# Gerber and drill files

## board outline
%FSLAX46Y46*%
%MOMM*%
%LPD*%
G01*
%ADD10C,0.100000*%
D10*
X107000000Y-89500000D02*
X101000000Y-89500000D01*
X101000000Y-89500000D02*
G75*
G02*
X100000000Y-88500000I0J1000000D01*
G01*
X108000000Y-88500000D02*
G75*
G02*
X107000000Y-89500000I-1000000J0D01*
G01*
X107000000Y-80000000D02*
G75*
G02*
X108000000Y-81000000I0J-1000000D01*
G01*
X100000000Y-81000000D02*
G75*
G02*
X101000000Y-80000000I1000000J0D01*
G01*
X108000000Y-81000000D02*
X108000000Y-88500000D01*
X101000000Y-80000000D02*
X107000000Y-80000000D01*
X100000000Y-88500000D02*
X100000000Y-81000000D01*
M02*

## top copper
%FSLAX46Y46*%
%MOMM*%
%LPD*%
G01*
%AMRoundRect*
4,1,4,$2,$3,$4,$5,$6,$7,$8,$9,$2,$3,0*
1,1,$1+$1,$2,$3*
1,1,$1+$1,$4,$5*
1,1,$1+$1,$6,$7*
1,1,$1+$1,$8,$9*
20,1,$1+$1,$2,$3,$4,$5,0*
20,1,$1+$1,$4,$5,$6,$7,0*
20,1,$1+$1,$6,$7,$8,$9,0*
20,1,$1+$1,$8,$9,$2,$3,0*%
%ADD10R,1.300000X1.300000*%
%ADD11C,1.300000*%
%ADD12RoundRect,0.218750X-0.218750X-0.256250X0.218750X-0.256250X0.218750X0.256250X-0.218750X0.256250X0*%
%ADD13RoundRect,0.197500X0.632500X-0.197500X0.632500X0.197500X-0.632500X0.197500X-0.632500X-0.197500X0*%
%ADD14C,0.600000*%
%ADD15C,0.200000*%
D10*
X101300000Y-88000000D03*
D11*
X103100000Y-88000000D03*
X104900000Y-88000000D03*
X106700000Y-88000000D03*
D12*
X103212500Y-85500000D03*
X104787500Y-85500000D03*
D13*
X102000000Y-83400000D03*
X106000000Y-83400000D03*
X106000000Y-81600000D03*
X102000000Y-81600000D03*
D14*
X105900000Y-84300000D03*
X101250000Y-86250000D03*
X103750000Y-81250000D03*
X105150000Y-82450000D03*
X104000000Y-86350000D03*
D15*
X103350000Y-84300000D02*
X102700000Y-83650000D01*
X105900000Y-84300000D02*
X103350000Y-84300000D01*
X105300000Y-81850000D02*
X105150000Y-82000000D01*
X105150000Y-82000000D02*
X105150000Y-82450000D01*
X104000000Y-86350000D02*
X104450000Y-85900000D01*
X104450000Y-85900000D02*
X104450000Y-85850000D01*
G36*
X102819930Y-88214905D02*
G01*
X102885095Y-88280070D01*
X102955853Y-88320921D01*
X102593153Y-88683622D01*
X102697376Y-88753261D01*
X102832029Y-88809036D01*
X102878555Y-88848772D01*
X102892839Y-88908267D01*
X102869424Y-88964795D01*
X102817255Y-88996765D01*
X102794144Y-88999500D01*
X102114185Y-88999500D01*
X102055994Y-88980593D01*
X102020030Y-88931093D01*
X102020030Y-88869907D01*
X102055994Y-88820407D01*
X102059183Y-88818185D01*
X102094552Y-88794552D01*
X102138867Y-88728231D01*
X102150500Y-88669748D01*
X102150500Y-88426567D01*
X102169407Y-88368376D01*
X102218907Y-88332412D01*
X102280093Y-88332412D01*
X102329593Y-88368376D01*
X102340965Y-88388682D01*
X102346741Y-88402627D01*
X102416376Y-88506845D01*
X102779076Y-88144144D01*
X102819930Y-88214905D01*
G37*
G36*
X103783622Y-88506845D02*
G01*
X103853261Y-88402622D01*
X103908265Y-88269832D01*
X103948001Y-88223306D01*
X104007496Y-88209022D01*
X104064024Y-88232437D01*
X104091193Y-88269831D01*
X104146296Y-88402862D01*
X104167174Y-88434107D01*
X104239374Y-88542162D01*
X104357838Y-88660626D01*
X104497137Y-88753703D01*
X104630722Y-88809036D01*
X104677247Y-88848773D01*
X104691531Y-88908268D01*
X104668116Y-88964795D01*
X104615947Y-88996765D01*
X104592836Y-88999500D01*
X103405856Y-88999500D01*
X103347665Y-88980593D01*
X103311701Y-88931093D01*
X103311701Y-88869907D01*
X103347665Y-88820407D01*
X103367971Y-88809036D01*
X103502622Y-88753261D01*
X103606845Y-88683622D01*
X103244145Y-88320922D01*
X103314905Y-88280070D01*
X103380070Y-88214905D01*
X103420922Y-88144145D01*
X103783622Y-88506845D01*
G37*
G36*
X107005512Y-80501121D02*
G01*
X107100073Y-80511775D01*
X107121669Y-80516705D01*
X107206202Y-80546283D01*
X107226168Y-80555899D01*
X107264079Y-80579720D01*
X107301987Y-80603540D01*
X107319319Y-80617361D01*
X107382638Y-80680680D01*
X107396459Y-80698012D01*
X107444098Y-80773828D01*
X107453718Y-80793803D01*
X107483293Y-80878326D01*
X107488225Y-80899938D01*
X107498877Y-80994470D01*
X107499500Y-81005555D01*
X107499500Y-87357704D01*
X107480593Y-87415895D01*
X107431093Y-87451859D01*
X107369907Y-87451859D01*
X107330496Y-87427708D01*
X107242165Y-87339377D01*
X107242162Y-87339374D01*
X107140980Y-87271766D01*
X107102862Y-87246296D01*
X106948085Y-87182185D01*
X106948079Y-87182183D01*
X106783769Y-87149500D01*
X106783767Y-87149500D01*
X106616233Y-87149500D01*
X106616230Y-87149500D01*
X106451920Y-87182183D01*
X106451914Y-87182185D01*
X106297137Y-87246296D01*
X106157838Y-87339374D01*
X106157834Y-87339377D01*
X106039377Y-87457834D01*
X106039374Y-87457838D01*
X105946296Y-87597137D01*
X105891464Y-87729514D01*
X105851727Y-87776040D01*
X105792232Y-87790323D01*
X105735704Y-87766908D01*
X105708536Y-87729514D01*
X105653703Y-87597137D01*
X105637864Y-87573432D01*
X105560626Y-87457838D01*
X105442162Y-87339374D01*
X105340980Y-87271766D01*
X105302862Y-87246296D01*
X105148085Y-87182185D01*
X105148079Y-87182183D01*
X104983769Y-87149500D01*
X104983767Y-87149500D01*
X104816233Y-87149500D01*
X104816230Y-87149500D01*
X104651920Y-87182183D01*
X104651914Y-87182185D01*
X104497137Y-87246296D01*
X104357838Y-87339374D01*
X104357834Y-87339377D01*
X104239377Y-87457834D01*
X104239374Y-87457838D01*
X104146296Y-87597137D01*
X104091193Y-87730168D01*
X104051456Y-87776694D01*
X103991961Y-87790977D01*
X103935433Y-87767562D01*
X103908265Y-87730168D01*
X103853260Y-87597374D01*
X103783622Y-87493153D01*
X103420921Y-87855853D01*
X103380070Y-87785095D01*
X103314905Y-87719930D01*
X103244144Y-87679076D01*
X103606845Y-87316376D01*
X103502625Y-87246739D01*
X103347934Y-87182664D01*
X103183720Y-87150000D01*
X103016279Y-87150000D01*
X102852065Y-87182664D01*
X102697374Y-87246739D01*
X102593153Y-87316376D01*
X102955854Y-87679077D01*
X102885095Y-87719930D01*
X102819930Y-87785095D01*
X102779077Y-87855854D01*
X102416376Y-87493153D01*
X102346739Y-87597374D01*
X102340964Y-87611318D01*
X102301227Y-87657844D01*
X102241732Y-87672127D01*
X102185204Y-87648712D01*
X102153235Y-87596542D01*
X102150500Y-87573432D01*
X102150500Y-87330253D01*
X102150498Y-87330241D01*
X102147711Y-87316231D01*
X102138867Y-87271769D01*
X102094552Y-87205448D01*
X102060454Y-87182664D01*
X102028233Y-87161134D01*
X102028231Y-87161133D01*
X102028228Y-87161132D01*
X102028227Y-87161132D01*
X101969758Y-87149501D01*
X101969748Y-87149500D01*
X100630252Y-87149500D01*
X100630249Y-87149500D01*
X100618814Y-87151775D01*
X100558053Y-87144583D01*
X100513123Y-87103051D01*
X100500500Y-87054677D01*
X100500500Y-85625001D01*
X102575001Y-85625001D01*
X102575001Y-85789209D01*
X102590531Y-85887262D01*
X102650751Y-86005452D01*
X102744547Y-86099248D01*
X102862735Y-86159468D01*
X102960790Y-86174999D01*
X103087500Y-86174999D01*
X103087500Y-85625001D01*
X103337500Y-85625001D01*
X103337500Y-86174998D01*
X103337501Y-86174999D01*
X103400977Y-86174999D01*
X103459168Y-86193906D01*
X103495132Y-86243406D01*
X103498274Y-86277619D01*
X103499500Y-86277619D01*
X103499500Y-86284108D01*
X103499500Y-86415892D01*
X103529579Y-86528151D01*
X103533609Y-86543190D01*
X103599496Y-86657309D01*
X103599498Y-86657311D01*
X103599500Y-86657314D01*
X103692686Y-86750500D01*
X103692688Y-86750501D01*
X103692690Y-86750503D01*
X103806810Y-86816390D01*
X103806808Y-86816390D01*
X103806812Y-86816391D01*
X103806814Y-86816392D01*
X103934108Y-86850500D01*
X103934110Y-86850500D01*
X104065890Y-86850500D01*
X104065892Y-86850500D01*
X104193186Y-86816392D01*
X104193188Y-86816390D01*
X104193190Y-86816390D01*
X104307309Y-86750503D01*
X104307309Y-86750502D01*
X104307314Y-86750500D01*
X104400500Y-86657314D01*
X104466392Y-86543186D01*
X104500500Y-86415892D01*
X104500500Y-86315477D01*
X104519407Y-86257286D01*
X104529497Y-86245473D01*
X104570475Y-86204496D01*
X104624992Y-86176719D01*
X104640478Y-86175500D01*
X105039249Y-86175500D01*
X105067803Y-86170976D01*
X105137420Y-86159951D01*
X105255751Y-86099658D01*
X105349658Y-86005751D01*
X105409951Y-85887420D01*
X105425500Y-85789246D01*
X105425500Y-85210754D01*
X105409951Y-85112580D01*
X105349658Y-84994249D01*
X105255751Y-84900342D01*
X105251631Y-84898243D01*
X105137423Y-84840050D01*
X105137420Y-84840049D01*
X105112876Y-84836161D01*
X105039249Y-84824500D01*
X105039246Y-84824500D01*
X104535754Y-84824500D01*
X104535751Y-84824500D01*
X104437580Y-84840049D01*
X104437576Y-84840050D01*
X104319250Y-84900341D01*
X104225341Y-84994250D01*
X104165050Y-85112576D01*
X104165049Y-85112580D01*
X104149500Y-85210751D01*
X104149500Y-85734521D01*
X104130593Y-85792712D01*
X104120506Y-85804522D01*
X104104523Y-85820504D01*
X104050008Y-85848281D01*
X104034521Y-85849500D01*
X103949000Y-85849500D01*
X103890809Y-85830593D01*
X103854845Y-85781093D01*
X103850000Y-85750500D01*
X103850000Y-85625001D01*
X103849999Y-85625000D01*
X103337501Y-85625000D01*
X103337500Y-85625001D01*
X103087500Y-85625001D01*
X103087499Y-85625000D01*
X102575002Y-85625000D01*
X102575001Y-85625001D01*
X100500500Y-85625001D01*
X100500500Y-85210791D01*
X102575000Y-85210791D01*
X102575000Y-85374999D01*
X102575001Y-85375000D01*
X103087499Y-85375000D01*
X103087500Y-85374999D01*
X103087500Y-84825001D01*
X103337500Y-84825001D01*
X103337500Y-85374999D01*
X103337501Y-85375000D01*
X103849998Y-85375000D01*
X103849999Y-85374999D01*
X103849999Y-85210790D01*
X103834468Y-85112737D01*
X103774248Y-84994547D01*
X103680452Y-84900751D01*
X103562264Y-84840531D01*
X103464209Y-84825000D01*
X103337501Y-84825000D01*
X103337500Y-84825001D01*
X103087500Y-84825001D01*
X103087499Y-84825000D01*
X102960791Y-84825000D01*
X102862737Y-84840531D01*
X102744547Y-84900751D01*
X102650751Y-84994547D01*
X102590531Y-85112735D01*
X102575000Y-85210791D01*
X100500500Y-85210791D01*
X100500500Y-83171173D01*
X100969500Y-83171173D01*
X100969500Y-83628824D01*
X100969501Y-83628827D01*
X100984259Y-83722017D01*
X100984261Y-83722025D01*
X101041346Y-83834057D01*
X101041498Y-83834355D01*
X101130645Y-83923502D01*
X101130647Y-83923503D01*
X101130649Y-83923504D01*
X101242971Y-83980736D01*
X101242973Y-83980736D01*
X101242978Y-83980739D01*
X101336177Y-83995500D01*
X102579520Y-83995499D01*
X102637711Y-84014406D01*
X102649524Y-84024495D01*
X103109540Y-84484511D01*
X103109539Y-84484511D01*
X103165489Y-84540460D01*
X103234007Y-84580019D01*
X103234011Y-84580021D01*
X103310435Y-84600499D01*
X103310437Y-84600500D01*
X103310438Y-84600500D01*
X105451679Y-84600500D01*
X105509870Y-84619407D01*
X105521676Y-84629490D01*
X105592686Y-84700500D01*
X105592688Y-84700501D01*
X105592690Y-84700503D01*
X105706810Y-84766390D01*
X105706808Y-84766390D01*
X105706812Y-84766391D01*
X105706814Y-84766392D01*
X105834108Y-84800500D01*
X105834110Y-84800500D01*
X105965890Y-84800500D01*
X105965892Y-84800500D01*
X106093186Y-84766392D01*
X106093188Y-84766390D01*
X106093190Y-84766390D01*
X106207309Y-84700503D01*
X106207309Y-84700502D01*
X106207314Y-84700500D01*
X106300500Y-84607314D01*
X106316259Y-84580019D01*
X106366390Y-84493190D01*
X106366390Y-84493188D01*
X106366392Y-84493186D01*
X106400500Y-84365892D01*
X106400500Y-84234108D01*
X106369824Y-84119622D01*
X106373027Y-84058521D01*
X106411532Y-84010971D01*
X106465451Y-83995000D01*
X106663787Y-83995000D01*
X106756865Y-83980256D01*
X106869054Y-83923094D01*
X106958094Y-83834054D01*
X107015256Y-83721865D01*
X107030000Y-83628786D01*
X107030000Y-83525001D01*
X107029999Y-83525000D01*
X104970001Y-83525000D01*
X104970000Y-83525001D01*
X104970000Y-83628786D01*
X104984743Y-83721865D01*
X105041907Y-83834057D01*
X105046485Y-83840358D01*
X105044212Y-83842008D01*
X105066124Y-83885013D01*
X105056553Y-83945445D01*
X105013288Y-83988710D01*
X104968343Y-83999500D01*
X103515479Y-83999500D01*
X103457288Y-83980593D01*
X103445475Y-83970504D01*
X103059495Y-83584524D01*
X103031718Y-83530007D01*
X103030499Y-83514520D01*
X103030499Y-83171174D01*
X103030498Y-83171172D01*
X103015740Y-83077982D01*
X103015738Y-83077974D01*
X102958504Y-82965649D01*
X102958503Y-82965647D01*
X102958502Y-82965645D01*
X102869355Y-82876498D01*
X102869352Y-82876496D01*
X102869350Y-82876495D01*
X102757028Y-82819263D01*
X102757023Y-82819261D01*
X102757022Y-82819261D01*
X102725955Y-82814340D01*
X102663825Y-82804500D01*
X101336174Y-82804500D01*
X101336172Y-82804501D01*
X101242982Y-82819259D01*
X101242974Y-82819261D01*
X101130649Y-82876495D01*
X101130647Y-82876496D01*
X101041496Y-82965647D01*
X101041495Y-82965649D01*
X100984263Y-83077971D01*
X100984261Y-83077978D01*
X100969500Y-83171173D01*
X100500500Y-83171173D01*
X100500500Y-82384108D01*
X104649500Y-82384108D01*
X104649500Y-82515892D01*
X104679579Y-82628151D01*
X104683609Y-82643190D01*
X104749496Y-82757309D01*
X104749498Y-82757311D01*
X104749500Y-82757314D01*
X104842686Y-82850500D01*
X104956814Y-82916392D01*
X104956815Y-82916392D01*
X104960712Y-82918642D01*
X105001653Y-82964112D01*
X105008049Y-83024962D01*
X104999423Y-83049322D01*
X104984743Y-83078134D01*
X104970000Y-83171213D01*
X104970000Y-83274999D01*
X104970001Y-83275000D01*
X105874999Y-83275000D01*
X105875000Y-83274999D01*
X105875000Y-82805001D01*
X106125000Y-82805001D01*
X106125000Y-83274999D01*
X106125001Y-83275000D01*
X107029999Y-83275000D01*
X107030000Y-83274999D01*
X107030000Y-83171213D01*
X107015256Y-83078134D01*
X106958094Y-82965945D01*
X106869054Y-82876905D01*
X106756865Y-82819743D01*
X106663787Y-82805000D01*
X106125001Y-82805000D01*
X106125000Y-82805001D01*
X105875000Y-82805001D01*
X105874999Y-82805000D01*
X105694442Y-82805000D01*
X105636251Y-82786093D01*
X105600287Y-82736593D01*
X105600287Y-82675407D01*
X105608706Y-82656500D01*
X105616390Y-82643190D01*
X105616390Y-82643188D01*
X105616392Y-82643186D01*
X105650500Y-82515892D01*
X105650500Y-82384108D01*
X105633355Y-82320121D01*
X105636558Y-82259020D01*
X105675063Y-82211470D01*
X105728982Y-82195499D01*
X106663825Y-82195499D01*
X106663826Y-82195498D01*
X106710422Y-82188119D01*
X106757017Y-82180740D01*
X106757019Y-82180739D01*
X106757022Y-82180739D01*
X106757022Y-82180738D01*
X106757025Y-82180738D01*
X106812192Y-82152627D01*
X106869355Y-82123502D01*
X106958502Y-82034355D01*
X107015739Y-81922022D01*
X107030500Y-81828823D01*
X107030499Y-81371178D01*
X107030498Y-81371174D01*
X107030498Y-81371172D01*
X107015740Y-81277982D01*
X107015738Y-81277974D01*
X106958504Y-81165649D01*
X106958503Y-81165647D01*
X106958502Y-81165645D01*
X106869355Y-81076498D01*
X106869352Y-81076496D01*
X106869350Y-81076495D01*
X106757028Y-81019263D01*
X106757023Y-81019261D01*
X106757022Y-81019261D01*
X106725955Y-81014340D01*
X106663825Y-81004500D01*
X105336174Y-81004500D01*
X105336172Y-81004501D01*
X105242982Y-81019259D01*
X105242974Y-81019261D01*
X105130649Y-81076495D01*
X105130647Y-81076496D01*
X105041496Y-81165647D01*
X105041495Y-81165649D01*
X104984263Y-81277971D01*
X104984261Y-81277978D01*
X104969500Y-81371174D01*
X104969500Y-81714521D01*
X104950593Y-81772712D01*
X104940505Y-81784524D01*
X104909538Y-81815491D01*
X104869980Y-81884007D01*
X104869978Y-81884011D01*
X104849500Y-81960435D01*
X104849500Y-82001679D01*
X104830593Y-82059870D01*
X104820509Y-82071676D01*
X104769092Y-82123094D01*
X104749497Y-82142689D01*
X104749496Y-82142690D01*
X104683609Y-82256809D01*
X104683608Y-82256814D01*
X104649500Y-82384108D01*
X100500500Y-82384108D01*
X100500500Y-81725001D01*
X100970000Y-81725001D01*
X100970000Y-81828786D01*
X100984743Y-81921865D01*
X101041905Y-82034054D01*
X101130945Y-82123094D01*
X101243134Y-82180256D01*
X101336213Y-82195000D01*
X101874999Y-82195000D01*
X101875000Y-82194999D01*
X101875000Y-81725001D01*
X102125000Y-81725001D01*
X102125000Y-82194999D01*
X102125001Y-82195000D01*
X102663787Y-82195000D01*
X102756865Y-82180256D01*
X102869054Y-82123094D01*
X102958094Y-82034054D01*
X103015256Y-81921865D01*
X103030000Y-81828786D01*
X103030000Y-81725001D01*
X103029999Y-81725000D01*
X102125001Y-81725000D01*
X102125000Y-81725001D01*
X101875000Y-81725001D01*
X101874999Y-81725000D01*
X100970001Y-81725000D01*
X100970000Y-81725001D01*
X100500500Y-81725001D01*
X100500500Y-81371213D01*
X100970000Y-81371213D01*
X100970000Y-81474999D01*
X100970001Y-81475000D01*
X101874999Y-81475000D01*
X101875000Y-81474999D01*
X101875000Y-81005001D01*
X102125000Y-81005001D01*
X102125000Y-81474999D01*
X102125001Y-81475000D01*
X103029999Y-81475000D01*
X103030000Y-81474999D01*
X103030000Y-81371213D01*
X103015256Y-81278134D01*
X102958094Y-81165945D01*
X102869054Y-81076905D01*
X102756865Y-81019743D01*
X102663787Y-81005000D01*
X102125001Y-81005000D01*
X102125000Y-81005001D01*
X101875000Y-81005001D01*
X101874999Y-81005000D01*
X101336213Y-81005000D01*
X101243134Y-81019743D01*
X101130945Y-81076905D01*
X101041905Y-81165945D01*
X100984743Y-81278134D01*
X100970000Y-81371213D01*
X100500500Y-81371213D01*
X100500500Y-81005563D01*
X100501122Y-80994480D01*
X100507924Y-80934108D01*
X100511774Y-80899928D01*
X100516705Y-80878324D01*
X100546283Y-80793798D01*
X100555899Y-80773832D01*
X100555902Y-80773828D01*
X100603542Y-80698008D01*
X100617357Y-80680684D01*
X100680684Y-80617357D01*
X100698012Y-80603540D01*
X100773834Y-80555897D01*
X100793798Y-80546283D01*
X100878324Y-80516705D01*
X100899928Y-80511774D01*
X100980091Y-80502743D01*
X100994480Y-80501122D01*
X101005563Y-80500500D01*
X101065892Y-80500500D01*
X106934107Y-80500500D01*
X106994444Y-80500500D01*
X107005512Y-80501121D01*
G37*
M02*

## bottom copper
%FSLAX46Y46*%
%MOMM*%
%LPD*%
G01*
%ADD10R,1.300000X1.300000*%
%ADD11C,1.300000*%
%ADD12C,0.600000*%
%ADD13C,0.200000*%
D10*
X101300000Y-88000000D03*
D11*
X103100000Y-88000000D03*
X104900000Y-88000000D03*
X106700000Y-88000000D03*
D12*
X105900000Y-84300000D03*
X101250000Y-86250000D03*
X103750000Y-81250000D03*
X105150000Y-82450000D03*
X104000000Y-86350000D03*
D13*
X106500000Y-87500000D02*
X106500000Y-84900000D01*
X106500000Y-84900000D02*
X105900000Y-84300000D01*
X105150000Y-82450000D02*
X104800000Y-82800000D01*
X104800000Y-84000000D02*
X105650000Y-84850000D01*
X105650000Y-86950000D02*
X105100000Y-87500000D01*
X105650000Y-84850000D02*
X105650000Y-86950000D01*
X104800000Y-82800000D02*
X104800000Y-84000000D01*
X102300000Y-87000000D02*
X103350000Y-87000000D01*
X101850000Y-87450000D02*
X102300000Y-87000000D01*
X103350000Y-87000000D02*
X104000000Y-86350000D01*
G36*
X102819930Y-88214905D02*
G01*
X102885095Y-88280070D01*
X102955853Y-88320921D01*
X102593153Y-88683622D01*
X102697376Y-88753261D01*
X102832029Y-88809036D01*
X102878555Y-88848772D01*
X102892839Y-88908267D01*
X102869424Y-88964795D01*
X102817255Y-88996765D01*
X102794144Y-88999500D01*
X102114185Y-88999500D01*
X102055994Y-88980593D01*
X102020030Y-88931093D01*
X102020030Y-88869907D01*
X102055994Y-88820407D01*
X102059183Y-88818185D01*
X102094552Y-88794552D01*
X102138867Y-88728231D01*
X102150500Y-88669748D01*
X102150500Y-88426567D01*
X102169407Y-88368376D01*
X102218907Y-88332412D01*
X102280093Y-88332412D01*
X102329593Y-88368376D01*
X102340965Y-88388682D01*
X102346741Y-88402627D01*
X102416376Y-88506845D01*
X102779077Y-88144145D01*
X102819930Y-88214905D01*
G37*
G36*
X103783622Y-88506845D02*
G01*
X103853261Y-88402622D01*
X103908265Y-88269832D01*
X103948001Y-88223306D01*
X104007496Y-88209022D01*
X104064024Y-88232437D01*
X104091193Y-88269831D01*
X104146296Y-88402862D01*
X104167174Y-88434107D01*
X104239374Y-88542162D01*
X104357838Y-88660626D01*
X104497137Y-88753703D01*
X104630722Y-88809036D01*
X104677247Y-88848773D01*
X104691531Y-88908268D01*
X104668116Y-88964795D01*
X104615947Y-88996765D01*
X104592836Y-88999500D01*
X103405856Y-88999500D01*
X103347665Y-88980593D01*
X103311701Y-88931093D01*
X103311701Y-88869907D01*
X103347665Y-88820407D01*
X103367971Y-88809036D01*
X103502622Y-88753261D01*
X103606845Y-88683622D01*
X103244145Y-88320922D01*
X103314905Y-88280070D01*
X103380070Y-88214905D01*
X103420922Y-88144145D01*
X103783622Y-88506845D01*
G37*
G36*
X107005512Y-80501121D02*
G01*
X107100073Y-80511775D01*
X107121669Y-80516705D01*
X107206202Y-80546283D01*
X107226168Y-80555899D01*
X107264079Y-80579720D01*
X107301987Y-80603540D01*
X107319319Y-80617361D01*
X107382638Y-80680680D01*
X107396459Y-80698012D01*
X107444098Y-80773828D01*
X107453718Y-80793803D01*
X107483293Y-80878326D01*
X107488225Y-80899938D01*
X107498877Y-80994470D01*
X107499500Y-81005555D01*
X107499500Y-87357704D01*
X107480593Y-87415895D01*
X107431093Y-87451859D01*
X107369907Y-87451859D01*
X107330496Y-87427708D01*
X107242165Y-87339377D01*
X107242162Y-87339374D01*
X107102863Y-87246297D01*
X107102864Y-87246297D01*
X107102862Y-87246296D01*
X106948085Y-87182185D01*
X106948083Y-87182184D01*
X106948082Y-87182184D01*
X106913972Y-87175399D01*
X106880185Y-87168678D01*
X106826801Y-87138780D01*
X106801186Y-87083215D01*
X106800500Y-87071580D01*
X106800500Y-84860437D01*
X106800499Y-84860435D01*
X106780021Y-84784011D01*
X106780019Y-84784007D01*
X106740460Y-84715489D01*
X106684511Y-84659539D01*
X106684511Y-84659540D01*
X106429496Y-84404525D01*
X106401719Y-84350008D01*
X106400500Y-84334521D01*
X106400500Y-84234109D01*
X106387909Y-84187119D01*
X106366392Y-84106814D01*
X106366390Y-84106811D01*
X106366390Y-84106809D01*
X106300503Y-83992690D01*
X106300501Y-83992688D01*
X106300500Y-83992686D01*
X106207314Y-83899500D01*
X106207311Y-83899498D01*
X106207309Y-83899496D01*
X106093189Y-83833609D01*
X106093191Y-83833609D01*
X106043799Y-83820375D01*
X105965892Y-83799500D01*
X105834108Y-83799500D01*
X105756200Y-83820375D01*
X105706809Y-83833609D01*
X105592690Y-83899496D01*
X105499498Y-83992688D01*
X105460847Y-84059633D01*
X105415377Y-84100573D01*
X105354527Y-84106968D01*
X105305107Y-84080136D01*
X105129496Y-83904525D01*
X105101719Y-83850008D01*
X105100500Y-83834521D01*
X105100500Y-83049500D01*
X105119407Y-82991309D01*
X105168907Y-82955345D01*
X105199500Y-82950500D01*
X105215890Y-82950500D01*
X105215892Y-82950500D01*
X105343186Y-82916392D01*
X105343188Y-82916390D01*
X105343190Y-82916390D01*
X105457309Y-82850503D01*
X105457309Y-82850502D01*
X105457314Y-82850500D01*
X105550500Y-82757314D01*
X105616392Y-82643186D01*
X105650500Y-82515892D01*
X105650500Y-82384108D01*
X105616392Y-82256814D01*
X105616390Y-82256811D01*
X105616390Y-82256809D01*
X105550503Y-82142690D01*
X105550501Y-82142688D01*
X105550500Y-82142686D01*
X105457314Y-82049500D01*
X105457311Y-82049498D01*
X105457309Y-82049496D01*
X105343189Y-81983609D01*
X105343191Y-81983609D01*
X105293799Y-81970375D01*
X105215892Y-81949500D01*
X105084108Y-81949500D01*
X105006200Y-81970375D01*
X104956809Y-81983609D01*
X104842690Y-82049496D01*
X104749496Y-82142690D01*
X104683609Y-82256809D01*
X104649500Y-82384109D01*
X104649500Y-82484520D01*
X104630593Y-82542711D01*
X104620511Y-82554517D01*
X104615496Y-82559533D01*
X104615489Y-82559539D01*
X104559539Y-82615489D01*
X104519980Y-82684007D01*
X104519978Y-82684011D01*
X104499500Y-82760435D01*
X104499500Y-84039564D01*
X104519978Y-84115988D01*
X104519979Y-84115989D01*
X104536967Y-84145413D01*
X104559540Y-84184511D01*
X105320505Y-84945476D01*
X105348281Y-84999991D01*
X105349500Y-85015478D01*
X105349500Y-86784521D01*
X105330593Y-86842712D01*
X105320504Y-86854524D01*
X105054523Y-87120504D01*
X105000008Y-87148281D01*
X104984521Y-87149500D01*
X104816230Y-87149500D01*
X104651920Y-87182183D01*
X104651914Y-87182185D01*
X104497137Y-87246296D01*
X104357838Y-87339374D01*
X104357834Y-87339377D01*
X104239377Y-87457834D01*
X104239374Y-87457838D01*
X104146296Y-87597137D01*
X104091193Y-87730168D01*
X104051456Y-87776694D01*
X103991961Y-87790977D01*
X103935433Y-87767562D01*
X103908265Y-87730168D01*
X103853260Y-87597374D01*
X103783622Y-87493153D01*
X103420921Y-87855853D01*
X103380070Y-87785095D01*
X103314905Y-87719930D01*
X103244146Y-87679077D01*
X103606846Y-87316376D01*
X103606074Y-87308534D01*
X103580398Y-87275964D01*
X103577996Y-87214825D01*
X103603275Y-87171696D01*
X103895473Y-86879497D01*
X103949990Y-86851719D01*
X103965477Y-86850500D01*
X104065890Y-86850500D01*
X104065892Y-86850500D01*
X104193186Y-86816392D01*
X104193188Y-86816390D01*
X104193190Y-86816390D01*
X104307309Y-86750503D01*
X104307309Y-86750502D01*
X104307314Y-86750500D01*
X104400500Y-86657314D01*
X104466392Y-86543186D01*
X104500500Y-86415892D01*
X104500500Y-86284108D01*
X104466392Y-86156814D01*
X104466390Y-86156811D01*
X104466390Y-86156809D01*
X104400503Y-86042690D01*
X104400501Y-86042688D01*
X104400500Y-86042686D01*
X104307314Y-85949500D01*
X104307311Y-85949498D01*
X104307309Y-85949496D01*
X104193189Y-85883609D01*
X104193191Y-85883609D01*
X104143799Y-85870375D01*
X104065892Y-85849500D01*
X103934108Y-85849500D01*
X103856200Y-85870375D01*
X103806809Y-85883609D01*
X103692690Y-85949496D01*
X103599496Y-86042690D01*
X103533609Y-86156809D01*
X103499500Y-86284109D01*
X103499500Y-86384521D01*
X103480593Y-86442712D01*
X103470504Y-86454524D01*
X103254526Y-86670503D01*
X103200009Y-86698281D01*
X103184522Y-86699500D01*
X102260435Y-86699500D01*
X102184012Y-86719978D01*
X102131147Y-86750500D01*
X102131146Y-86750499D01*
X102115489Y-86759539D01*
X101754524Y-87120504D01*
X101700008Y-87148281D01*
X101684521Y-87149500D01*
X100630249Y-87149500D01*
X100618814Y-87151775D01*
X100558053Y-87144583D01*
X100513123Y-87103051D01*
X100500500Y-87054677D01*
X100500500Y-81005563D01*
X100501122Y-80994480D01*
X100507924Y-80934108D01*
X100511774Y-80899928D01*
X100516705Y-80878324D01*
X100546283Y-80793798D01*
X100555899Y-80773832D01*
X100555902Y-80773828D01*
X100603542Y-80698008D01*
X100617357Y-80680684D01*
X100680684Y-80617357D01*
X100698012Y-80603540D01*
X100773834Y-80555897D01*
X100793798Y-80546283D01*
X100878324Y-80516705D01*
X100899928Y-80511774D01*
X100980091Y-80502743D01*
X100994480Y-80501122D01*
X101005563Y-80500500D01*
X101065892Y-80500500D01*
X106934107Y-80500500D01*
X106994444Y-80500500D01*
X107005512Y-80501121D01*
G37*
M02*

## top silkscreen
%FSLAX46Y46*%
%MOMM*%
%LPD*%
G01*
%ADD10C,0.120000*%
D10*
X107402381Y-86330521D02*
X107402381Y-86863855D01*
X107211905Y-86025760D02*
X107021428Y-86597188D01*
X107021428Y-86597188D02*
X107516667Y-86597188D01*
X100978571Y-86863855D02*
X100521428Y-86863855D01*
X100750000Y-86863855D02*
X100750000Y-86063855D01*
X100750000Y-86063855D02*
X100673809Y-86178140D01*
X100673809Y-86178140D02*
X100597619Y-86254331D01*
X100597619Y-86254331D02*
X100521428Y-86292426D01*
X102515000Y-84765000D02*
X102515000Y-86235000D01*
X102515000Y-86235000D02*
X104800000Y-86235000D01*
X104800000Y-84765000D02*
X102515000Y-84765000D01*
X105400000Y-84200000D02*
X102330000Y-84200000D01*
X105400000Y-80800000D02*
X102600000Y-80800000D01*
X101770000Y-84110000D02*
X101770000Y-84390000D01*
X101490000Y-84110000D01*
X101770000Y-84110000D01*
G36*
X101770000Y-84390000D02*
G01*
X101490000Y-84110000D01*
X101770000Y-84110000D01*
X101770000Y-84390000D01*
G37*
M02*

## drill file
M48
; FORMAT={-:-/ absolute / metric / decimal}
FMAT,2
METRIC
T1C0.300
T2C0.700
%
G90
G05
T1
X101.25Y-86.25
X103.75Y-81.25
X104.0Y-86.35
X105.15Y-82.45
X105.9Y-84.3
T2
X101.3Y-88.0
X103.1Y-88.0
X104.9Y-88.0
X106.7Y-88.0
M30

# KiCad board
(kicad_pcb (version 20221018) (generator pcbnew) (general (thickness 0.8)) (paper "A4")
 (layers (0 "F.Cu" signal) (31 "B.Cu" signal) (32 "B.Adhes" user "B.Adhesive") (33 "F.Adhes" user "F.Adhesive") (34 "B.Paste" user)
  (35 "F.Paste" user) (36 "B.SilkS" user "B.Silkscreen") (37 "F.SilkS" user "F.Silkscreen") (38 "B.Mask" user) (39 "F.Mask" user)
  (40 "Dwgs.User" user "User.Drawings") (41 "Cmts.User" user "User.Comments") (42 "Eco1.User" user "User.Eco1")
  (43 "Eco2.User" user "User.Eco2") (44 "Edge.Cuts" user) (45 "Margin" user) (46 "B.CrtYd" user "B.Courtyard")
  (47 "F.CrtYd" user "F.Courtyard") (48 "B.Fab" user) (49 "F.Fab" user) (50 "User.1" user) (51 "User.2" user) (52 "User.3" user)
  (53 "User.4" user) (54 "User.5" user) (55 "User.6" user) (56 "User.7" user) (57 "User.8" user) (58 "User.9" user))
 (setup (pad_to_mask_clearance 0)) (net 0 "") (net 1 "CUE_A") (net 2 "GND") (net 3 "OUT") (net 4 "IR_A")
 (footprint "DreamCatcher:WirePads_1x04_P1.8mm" (layer "F.Cu") (at 104 88)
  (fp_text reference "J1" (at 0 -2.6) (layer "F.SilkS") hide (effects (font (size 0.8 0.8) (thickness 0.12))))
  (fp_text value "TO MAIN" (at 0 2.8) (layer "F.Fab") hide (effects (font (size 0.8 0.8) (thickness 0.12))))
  (pad "1" thru_hole rect (at -2.7 0) (size 1.3 1.3) (drill 0.7) (layers "*.Cu" "*.Mask") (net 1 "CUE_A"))
  (pad "2" thru_hole circle (at -0.9 0) (size 1.3 1.3) (drill 0.7) (layers "*.Cu" "*.Mask") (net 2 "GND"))
  (pad "3" thru_hole circle (at 0.9 0) (size 1.3 1.3) (drill 0.7) (layers "*.Cu" "*.Mask") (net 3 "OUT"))
  (pad "4" thru_hole circle (at 2.7 0) (size 1.3 1.3) (drill 0.7) (layers "*.Cu" "*.Mask") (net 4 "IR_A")))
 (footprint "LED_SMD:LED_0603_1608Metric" (layer "F.Cu") (at 104 85.5)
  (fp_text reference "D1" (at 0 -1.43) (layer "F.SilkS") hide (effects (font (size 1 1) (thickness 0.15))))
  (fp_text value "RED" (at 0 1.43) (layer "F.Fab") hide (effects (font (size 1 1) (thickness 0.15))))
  (fp_line (start -1.485 -0.735) (end -1.485 0.735) (stroke (width 0.12) (type solid)) (layer "F.SilkS"))
  (fp_line (start -1.485 0.735) (end 0.8 0.735) (stroke (width 0.12) (type solid)) (layer "F.SilkS"))
  (fp_line (start 0.8 -0.735) (end -1.485 -0.735) (stroke (width 0.12) (type solid)) (layer "F.SilkS"))
  (pad "1" smd roundrect (at -0.7875 0) (size 0.875 0.95) (layers "F.Cu" "F.Paste" "F.Mask") (roundrect_rratio 0.25) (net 2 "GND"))
  (pad "2" smd roundrect (at 0.7875 0) (size 0.875 0.95) (layers "F.Cu" "F.Paste" "F.Mask") (roundrect_rratio 0.25) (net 1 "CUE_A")))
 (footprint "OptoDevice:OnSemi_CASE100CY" (layer "F.Cu") (at 104 82.5 90)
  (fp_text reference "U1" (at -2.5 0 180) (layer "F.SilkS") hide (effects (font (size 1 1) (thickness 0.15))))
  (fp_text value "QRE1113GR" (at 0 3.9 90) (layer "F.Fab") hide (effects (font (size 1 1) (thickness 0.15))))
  (fp_line (start -1.7 1.4) (end -1.7 -1.67) (stroke (width 0.12) (type solid)) (layer "F.SilkS"))
  (fp_line (start 1.7 1.4) (end 1.7 -1.4) (stroke (width 0.12) (type solid)) (layer "F.SilkS"))
  (fp_poly
   (pts (xy -1.61 -2.23) (xy -1.89 -2.23) (xy -1.61 -2.51) (xy -1.61 -2.23)) (stroke (width 0.12) (type solid)) (fill solid)
   (layer "F.SilkS"))
  (pad "1" smd roundrect (at -0.9 -2 90) (size 0.79 1.66) (layers "F.Cu" "F.Paste" "F.Mask") (roundrect_rratio 0.25) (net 4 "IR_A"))
  (pad "2" smd roundrect (at -0.9 2 90) (size 0.79 1.66) (layers "F.Cu" "F.Paste" "F.Mask") (roundrect_rratio 0.25) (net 2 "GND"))
  (pad "3" smd roundrect (at 0.9 2 90) (size 0.79 1.66) (layers "F.Cu" "F.Paste" "F.Mask") (roundrect_rratio 0.25) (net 3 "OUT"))
  (pad "4" smd roundrect (at 0.9 -2 90) (size 0.79 1.66) (layers "F.Cu" "F.Paste" "F.Mask") (roundrect_rratio 0.25) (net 2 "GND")))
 (gr_line (start 107 89.5) (end 101 89.5) (stroke (width 0.1) (type default)) (layer "Edge.Cuts"))
 (gr_arc (start 101 89.5) (mid 100.292893 89.207106) (end 100 88.5) (stroke (width 0.1) (type default)) (layer "Edge.Cuts"))
 (gr_arc (start 108 88.5) (mid 107.707106 89.207106) (end 107 89.5) (stroke (width 0.1) (type default)) (layer "Edge.Cuts"))
 (gr_arc (start 107 80) (mid 107.707106 80.292893) (end 108 81) (stroke (width 0.1) (type default)) (layer "Edge.Cuts"))
 (gr_arc (start 100 81) (mid 100.292893 80.292893) (end 101 80) (stroke (width 0.1) (type default)) (layer "Edge.Cuts"))
 (gr_line (start 108 81) (end 108 88.5) (stroke (width 0.1) (type default)) (layer "Edge.Cuts"))
 (gr_line (start 101 80) (end 107 80) (stroke (width 0.1) (type default)) (layer "Edge.Cuts"))
 (gr_line (start 100 88.5) (end 100 81) (stroke (width 0.1) (type default)) (layer "Edge.Cuts"))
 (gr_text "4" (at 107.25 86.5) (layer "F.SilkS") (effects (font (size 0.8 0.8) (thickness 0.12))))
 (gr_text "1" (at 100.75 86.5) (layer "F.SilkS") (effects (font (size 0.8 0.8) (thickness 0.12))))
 (segment (start 103.35 84.3) (end 102.7 83.65) (width 0.2) (layer "F.Cu") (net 4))
 (segment (start 105.9 84.3) (end 103.35 84.3) (width 0.2) (layer "F.Cu") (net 4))
 (via (at 105.9 84.3) (size 0.6) (drill 0.3) (layers "F.Cu" "B.Cu") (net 4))
 (segment (start 106.5 87.5) (end 106.5 84.9) (width 0.2) (layer "B.Cu") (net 4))
 (segment (start 106.5 84.9) (end 105.9 84.3) (width 0.2) (layer "B.Cu") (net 4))
 (via (at 101.25 86.25) (size 0.6) (drill 0.3) (layers "F.Cu" "B.Cu") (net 2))
 (via (at 103.75 81.25) (size 0.6) (drill 0.3) (layers "F.Cu" "B.Cu") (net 2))
 (segment (start 105.3 81.85) (end 105.15 82) (width 0.2) (layer "F.Cu") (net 3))
 (segment (start 105.15 82) (end 105.15 82.45) (width 0.2) (layer "F.Cu") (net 3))
 (via (at 105.15 82.45) (size 0.6) (drill 0.3) (layers "F.Cu" "B.Cu") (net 3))
 (segment (start 105.15 82.45) (end 104.8 82.8) (width 0.2) (layer "B.Cu") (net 3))
 (segment (start 104.8 84) (end 105.65 84.85) (width 0.2) (layer "B.Cu") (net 3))
 (segment (start 105.65 86.95) (end 105.1 87.5) (width 0.2) (layer "B.Cu") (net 3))
 (segment (start 105.65 84.85) (end 105.65 86.95) (width 0.2) (layer "B.Cu") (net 3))
 (segment (start 104.8 82.8) (end 104.8 84) (width 0.2) (layer "B.Cu") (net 3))
 (segment (start 104 86.35) (end 104.45 85.9) (width 0.2) (layer "F.Cu") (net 1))
 (segment (start 104.45 85.9) (end 104.45 85.85) (width 0.2) (layer "F.Cu") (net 1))
 (via (at 104 86.35) (size 0.6) (drill 0.3) (layers "F.Cu" "B.Cu") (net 1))
 (segment (start 102.3 87) (end 103.35 87) (width 0.2) (layer "B.Cu") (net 1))
 (segment (start 101.85 87.45) (end 102.3 87) (width 0.2) (layer "B.Cu") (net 1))
 (segment (start 103.35 87) (end 104 86.35) (width 0.2) (layer "B.Cu") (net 1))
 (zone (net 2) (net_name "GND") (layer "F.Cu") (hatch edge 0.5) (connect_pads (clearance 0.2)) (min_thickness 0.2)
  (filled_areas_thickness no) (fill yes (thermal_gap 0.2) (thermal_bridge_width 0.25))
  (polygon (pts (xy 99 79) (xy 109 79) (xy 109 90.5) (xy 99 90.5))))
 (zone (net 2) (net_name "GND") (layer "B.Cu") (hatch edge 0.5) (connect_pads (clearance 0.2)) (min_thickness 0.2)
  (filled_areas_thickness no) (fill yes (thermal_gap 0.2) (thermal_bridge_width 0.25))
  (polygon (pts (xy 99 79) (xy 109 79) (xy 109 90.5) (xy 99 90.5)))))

